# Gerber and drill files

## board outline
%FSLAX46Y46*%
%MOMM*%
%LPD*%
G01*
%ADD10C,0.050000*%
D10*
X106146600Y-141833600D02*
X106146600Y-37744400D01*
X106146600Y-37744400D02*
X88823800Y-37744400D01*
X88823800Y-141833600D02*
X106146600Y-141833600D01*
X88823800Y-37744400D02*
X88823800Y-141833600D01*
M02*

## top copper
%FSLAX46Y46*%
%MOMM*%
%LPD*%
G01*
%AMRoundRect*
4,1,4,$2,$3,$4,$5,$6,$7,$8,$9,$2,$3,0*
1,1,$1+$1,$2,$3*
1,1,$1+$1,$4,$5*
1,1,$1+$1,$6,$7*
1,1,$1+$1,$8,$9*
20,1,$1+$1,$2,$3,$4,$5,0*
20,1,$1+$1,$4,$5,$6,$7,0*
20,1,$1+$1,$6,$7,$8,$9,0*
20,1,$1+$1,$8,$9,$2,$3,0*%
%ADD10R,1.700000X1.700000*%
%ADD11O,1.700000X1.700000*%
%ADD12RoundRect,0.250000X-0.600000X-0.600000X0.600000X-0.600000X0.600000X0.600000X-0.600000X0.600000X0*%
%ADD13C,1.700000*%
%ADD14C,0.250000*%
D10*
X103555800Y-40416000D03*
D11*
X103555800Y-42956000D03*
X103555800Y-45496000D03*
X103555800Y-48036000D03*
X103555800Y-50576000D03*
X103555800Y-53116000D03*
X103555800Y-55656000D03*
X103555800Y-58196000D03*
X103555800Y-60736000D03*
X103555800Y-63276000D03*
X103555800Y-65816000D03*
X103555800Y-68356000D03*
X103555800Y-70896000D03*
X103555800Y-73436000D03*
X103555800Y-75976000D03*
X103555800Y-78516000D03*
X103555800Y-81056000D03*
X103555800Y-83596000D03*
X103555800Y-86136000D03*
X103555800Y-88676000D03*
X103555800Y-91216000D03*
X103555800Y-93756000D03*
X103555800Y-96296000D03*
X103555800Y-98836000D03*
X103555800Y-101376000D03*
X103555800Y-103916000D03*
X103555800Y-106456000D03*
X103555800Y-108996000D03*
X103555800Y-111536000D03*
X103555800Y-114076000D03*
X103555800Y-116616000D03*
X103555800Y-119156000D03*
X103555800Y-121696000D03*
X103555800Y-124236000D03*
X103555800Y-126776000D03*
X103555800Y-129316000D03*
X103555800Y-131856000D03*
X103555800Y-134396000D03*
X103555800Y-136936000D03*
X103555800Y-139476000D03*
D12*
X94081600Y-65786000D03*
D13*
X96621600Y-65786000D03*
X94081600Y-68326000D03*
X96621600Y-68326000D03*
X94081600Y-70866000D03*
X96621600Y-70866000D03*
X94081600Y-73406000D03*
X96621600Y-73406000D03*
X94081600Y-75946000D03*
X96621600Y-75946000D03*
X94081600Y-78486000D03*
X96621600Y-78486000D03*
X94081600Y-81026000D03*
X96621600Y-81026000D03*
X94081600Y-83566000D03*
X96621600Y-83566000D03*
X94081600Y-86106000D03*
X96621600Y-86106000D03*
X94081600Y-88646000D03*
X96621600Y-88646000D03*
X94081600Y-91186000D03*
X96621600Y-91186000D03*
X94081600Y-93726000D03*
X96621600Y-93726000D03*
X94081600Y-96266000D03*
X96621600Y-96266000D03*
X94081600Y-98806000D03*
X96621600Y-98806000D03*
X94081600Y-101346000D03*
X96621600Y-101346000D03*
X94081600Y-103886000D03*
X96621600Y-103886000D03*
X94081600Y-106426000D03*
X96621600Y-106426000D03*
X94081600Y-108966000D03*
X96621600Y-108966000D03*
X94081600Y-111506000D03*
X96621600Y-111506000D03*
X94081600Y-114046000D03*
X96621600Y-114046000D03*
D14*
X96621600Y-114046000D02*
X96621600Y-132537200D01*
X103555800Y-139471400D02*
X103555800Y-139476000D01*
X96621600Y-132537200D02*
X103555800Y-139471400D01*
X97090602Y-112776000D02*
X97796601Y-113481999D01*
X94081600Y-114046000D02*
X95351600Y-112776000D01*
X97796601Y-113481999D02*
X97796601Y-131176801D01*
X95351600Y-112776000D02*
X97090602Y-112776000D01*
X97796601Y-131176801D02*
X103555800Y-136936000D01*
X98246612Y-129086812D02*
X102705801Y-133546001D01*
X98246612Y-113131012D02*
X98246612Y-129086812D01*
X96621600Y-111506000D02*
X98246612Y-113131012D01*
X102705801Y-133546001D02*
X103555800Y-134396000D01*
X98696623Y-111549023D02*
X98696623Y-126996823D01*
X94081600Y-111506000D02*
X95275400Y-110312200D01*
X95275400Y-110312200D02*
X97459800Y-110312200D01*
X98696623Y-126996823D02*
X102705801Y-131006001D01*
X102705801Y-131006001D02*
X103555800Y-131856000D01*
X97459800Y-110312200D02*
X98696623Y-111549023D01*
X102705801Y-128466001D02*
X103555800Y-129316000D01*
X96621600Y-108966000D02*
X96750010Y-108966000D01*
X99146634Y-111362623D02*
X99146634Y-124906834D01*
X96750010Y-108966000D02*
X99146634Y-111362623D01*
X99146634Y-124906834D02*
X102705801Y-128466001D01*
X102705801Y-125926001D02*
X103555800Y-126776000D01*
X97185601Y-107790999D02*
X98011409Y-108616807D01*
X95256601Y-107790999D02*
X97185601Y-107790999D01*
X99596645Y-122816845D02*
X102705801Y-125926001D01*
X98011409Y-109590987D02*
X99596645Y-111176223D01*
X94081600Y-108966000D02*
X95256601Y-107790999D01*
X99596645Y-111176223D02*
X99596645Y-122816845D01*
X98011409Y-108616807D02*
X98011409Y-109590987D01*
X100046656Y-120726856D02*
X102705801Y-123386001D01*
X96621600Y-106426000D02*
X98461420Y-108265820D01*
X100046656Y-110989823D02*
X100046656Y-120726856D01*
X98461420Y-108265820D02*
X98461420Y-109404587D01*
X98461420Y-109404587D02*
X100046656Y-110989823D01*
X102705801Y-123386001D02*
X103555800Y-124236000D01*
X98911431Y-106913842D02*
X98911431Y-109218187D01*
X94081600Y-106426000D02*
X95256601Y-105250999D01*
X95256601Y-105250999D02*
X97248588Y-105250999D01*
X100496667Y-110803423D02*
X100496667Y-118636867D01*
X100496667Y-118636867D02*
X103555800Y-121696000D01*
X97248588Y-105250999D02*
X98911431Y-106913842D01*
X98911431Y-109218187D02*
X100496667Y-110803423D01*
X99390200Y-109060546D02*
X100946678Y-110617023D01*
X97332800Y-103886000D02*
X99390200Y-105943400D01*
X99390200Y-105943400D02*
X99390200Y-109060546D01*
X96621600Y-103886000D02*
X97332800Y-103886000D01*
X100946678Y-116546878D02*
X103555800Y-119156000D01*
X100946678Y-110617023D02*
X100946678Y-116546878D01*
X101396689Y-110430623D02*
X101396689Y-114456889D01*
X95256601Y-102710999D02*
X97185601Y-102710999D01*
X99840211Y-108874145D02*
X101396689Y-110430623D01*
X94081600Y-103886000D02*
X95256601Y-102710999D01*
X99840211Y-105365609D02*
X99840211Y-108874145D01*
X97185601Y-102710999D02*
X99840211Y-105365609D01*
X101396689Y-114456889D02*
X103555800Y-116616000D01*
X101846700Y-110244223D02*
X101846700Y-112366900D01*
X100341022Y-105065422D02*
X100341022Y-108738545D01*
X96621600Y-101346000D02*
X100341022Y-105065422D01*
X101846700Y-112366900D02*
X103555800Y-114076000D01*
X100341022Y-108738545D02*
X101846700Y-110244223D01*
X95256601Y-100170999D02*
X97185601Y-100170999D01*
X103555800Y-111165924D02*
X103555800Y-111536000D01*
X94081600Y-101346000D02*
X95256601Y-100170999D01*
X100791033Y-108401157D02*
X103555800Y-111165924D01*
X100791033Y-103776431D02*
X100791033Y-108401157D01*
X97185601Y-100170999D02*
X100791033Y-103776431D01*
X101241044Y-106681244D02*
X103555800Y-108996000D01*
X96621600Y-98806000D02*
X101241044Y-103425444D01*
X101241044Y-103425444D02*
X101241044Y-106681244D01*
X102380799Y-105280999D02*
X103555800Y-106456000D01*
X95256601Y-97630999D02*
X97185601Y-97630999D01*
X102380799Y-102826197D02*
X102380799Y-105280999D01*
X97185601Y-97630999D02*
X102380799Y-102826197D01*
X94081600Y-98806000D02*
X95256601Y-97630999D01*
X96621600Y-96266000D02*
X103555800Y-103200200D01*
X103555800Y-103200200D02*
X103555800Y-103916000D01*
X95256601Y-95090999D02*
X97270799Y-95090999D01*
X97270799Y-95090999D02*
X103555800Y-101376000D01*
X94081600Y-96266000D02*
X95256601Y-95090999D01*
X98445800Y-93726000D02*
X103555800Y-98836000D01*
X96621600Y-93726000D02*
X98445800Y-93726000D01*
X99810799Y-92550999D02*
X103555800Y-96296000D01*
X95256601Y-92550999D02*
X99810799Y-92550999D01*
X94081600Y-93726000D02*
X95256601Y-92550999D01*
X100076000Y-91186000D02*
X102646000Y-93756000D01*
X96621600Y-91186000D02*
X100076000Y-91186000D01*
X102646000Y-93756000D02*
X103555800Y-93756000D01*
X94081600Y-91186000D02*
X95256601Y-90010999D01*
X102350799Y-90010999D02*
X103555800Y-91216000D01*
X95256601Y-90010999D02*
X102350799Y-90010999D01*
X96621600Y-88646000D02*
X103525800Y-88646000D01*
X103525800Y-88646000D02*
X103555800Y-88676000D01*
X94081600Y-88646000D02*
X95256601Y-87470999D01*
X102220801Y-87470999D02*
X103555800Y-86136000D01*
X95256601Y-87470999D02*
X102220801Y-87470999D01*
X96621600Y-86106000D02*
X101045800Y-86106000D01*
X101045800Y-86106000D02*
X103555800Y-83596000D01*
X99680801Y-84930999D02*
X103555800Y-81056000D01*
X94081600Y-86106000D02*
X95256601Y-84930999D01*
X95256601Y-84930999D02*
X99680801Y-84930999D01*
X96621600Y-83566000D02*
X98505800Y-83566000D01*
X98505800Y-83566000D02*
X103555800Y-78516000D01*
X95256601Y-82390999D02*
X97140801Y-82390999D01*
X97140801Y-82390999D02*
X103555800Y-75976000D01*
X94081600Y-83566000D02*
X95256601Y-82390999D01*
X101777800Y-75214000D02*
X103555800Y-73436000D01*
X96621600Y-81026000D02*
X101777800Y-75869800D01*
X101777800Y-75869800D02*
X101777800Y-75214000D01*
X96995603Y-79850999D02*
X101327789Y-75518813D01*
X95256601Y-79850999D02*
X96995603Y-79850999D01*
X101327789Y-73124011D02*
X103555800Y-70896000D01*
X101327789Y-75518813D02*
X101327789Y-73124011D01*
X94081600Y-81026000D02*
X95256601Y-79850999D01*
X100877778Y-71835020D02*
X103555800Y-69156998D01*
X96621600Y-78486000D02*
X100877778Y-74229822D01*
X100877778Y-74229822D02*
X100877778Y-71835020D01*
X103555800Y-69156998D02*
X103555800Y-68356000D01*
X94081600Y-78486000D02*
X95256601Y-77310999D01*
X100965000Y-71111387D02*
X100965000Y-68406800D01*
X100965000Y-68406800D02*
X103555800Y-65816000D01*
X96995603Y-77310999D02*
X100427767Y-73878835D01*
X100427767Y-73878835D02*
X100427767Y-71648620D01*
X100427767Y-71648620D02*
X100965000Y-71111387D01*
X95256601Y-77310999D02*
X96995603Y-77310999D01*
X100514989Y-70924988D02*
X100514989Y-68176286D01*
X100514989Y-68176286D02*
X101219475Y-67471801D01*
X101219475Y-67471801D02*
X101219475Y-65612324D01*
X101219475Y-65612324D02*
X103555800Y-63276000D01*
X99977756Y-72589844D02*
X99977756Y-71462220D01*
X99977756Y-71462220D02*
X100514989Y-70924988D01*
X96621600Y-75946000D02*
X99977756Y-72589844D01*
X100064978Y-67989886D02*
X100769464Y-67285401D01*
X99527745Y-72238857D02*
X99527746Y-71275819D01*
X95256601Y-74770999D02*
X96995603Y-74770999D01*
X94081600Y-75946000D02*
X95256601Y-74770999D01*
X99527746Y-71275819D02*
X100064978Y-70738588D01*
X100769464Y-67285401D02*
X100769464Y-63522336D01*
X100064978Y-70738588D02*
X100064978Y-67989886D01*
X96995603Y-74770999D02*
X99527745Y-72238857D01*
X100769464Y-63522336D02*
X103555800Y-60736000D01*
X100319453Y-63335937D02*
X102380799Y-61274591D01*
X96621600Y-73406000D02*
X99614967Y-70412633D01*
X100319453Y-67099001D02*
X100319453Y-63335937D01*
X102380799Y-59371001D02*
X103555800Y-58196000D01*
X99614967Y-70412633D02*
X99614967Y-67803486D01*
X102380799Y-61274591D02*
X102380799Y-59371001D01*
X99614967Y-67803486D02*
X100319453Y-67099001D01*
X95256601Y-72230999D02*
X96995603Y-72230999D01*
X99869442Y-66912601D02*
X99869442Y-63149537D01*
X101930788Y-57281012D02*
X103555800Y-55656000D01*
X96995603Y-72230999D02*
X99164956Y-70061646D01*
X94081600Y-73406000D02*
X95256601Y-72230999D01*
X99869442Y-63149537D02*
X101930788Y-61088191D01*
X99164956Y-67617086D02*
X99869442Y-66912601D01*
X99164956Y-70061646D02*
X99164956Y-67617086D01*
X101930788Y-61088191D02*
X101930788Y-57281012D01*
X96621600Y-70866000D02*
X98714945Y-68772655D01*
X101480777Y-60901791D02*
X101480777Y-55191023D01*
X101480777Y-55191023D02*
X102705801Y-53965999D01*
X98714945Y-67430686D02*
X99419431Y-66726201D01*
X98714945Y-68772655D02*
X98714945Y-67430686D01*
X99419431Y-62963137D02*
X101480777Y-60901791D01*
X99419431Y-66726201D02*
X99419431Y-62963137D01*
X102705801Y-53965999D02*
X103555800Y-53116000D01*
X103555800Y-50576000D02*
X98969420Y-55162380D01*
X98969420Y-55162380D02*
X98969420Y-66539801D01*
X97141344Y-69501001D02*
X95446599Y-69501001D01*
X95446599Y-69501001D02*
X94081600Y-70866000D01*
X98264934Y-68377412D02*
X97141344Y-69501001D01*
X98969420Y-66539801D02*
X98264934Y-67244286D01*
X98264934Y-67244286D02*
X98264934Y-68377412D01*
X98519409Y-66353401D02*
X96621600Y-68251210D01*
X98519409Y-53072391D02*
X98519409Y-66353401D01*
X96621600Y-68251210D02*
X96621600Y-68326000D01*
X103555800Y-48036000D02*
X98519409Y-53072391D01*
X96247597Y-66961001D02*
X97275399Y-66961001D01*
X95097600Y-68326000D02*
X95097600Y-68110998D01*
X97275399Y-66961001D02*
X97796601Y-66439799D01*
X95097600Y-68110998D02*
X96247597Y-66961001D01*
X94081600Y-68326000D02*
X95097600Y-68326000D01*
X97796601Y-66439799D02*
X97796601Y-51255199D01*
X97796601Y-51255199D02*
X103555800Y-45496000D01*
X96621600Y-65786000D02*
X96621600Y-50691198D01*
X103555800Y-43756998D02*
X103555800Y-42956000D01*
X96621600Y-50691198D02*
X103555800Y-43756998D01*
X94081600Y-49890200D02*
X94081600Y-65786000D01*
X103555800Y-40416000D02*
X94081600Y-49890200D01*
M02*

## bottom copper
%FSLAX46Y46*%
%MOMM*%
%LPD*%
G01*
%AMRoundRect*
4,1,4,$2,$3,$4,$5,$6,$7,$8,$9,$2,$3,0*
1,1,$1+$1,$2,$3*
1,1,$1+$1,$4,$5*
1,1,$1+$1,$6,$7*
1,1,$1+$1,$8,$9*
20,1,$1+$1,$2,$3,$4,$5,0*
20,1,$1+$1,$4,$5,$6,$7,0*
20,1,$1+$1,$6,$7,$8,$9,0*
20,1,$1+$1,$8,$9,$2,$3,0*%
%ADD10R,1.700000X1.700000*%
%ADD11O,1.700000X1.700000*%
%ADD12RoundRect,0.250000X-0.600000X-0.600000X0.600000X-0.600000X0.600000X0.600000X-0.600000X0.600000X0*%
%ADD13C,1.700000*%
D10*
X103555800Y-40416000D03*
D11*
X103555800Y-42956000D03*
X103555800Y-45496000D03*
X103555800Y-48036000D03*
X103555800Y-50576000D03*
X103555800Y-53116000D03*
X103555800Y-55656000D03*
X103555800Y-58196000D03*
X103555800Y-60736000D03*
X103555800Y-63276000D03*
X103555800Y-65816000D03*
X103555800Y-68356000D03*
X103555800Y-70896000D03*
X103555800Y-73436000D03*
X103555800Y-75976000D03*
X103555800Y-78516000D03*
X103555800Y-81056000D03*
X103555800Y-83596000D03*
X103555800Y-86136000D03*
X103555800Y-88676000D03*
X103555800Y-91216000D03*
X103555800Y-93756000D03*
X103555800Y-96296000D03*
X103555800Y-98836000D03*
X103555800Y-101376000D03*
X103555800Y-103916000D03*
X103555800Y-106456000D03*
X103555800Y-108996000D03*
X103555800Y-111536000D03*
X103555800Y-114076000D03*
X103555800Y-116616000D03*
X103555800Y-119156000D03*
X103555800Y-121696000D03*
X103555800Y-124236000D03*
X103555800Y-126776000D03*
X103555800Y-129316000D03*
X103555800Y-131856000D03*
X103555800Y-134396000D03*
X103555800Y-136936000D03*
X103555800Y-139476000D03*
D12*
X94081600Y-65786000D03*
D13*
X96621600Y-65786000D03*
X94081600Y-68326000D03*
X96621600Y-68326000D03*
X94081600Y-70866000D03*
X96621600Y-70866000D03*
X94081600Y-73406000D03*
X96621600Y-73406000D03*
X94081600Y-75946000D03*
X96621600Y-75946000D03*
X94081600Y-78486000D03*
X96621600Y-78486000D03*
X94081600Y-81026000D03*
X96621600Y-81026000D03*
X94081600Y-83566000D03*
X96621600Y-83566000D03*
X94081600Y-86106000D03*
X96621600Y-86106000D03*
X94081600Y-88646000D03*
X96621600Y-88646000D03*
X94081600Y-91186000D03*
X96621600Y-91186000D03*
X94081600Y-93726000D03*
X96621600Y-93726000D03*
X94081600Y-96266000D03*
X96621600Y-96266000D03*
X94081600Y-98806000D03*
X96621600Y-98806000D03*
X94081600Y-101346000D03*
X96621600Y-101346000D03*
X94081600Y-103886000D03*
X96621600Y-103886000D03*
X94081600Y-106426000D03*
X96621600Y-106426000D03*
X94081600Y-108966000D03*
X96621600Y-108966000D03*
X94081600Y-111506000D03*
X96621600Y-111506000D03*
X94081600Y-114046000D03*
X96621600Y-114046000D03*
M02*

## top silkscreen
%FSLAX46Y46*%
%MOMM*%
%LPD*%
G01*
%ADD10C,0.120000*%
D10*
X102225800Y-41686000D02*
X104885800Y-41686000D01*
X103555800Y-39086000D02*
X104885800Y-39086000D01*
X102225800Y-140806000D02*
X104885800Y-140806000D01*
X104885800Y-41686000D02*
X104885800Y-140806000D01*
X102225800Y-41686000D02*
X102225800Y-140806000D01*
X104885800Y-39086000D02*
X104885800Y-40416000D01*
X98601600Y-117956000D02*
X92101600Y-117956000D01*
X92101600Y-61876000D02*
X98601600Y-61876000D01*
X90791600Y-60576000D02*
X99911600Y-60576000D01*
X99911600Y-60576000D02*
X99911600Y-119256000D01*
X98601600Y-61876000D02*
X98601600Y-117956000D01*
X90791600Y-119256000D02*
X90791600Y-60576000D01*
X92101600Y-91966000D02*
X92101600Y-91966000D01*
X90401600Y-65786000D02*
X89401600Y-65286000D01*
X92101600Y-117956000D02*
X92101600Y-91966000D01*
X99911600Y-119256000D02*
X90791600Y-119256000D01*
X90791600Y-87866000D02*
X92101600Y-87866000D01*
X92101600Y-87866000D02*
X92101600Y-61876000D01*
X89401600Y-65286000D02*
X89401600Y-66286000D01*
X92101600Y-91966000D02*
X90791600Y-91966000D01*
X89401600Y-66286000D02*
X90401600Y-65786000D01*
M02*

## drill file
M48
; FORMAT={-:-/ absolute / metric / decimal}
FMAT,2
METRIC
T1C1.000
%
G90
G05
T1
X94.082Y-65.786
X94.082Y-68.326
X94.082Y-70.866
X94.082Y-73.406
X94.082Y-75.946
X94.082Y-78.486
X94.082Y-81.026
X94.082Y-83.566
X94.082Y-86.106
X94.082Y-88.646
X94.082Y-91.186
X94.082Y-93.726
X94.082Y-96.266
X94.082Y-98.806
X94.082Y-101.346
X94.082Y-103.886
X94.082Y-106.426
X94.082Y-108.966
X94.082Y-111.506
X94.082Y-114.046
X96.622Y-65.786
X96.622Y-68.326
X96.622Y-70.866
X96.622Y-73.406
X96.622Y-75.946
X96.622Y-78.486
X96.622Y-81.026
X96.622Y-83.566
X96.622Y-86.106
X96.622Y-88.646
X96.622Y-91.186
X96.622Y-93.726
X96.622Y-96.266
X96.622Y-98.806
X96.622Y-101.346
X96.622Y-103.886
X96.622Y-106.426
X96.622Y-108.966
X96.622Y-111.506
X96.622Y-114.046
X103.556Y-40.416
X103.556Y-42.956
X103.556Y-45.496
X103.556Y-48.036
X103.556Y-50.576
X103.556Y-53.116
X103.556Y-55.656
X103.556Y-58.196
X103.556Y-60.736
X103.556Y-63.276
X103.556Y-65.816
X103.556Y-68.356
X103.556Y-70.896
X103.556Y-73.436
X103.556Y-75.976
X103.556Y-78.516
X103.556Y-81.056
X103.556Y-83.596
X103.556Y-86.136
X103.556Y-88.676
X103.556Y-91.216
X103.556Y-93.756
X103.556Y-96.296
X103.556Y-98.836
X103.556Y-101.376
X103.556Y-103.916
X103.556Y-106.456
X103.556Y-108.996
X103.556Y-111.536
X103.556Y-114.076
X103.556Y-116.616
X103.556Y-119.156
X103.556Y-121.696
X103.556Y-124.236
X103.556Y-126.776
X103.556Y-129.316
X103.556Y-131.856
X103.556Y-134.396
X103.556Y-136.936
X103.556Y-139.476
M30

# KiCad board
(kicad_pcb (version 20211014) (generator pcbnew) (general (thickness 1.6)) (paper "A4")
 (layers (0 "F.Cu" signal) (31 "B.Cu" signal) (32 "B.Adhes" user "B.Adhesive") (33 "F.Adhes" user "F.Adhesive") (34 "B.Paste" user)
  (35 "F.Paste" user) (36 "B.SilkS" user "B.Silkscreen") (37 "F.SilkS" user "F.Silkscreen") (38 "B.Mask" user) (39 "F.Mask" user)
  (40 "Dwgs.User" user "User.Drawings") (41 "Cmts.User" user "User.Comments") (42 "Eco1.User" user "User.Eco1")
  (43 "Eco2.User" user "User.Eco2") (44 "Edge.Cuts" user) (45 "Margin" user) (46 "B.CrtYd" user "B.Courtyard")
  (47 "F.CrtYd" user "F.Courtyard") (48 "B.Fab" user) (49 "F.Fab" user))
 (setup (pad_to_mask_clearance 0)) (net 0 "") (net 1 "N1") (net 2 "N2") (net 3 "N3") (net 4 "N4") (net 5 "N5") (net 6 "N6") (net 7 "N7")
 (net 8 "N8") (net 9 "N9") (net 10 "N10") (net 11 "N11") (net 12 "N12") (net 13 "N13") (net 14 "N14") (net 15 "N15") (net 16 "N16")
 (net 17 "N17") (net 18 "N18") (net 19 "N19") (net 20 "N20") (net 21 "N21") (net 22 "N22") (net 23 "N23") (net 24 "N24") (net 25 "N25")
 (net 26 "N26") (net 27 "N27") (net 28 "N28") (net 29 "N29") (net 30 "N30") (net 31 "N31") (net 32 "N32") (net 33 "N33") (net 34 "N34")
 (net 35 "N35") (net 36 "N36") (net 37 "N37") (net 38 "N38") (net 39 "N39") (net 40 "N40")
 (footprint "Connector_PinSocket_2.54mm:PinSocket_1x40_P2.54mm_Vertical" (layer "F.Cu") (at 103.5558 40.416)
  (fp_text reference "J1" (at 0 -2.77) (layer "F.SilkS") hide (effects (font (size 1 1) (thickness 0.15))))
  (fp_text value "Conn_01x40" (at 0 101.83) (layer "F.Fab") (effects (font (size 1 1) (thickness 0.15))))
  (fp_line (start -1.33 1.27) (end 1.33 1.27) (layer "F.SilkS") (width 0.12))
  (fp_line (start 0 -1.33) (end 1.33 -1.33) (layer "F.SilkS") (width 0.12))
  (fp_line (start -1.33 100.39) (end 1.33 100.39) (layer "F.SilkS") (width 0.12))
  (fp_line (start 1.33 1.27) (end 1.33 100.39) (layer "F.SilkS") (width 0.12))
  (fp_line (start -1.33 1.27) (end -1.33 100.39) (layer "F.SilkS") (width 0.12))
  (fp_line (start 1.33 -1.33) (end 1.33 0) (layer "F.SilkS") (width 0.12))
  (pad "1" thru_hole rect locked (at 0 0) (size 1.7 1.7) (drill 1) (layers *.Cu *.Mask) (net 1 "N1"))
  (pad "2" thru_hole oval locked (at 0 2.54) (size 1.7 1.7) (drill 1) (layers *.Cu *.Mask) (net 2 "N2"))
  (pad "3" thru_hole oval locked (at 0 5.08) (size 1.7 1.7) (drill 1) (layers *.Cu *.Mask) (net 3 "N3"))
  (pad "4" thru_hole oval locked (at 0 7.62) (size 1.7 1.7) (drill 1) (layers *.Cu *.Mask) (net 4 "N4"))
  (pad "5" thru_hole oval locked (at 0 10.16) (size 1.7 1.7) (drill 1) (layers *.Cu *.Mask) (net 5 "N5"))
  (pad "6" thru_hole oval locked (at 0 12.7) (size 1.7 1.7) (drill 1) (layers *.Cu *.Mask) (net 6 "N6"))
  (pad "7" thru_hole oval locked (at 0 15.24) (size 1.7 1.7) (drill 1) (layers *.Cu *.Mask) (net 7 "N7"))
  (pad "8" thru_hole oval locked (at 0 17.78) (size 1.7 1.7) (drill 1) (layers *.Cu *.Mask) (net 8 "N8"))
  (pad "9" thru_hole oval locked (at 0 20.32) (size 1.7 1.7) (drill 1) (layers *.Cu *.Mask) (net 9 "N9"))
  (pad "10" thru_hole oval locked (at 0 22.86) (size 1.7 1.7) (drill 1) (layers *.Cu *.Mask) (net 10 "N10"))
  (pad "11" thru_hole oval locked (at 0 25.4) (size 1.7 1.7) (drill 1) (layers *.Cu *.Mask) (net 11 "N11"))
  (pad "12" thru_hole oval locked (at 0 27.94) (size 1.7 1.7) (drill 1) (layers *.Cu *.Mask) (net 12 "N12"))
  (pad "13" thru_hole oval locked (at 0 30.48) (size 1.7 1.7) (drill 1) (layers *.Cu *.Mask) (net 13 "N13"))
  (pad "14" thru_hole oval locked (at 0 33.02) (size 1.7 1.7) (drill 1) (layers *.Cu *.Mask) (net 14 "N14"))
  (pad "15" thru_hole oval locked (at 0 35.56) (size 1.7 1.7) (drill 1) (layers *.Cu *.Mask) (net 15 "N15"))
  (pad "16" thru_hole oval locked (at 0 38.1) (size 1.7 1.7) (drill 1) (layers *.Cu *.Mask) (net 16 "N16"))
  (pad "17" thru_hole oval locked (at 0 40.64) (size 1.7 1.7) (drill 1) (layers *.Cu *.Mask) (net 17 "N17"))
  (pad "18" thru_hole oval locked (at 0 43.18) (size 1.7 1.7) (drill 1) (layers *.Cu *.Mask) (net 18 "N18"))
  (pad "19" thru_hole oval locked (at 0 45.72) (size 1.7 1.7) (drill 1) (layers *.Cu *.Mask) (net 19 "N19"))
  (pad "20" thru_hole oval locked (at 0 48.26) (size 1.7 1.7) (drill 1) (layers *.Cu *.Mask) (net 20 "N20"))
  (pad "21" thru_hole oval locked (at 0 50.8) (size 1.7 1.7) (drill 1) (layers *.Cu *.Mask) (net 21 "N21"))
  (pad "22" thru_hole oval locked (at 0 53.34) (size 1.7 1.7) (drill 1) (layers *.Cu *.Mask) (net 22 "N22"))
  (pad "23" thru_hole oval locked (at 0 55.88) (size 1.7 1.7) (drill 1) (layers *.Cu *.Mask) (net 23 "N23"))
  (pad "24" thru_hole oval locked (at 0 58.42) (size 1.7 1.7) (drill 1) (layers *.Cu *.Mask) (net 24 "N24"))
  (pad "25" thru_hole oval locked (at 0 60.96) (size 1.7 1.7) (drill 1) (layers *.Cu *.Mask) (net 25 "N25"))
  (pad "26" thru_hole oval locked (at 0 63.5) (size 1.7 1.7) (drill 1) (layers *.Cu *.Mask) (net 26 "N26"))
  (pad "27" thru_hole oval locked (at 0 66.04) (size 1.7 1.7) (drill 1) (layers *.Cu *.Mask) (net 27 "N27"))
  (pad "28" thru_hole oval locked (at 0 68.58) (size 1.7 1.7) (drill 1) (layers *.Cu *.Mask) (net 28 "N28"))
  (pad "29" thru_hole oval locked (at 0 71.12) (size 1.7 1.7) (drill 1) (layers *.Cu *.Mask) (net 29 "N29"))
  (pad "30" thru_hole oval locked (at 0 73.66) (size 1.7 1.7) (drill 1) (layers *.Cu *.Mask) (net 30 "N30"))
  (pad "31" thru_hole oval locked (at 0 76.2) (size 1.7 1.7) (drill 1) (layers *.Cu *.Mask) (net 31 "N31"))
  (pad "32" thru_hole oval locked (at 0 78.74) (size 1.7 1.7) (drill 1) (layers *.Cu *.Mask) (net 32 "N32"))
  (pad "33" thru_hole oval locked (at 0 81.28) (size 1.7 1.7) (drill 1) (layers *.Cu *.Mask) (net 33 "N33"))
  (pad "34" thru_hole oval locked (at 0 83.82) (size 1.7 1.7) (drill 1) (layers *.Cu *.Mask) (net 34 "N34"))
  (pad "35" thru_hole oval locked (at 0 86.36) (size 1.7 1.7) (drill 1) (layers *.Cu *.Mask) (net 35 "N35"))
  (pad "36" thru_hole oval locked (at 0 88.9) (size 1.7 1.7) (drill 1) (layers *.Cu *.Mask) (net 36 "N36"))
  (pad "37" thru_hole oval locked (at 0 91.44) (size 1.7 1.7) (drill 1) (layers *.Cu *.Mask) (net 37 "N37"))
  (pad "38" thru_hole oval locked (at 0 93.98) (size 1.7 1.7) (drill 1) (layers *.Cu *.Mask) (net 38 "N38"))
  (pad "39" thru_hole oval locked (at 0 96.52) (size 1.7 1.7) (drill 1) (layers *.Cu *.Mask) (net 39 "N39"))
  (pad "40" thru_hole oval locked (at 0 99.06) (size 1.7 1.7) (drill 1) (layers *.Cu *.Mask) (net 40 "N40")))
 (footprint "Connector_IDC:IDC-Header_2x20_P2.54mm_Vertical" (layer "F.Cu") (at 94.0816 65.786)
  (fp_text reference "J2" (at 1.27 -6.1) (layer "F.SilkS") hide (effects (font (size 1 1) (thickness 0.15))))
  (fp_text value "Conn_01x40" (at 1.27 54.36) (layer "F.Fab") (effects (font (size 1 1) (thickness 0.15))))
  (fp_line (start 4.52 52.17) (end -1.98 52.17) (layer "F.SilkS") (width 0.12))
  (fp_line (start -1.98 -3.91) (end 4.52 -3.91) (layer "F.SilkS") (width 0.12))
  (fp_line (start -3.29 -5.21) (end 5.83 -5.21) (layer "F.SilkS") (width 0.12))
  (fp_line (start 5.83 -5.21) (end 5.83 53.47) (layer "F.SilkS") (width 0.12))
  (fp_line (start 4.52 -3.91) (end 4.52 52.17) (layer "F.SilkS") (width 0.12))
  (fp_line (start -3.29 53.47) (end -3.29 -5.21) (layer "F.SilkS") (width 0.12))
  (fp_line (start -1.98 26.18) (end -1.98 26.18) (layer "F.SilkS") (width 0.12))
  (fp_line (start -3.68 0) (end -4.68 -0.5) (layer "F.SilkS") (width 0.12))
  (fp_line (start -1.98 52.17) (end -1.98 26.18) (layer "F.SilkS") (width 0.12))
  (fp_line (start 5.83 53.47) (end -3.29 53.47) (layer "F.SilkS") (width 0.12))
  (fp_line (start -3.29 22.08) (end -1.98 22.08) (layer "F.SilkS") (width 0.12))
  (fp_line (start -1.98 22.08) (end -1.98 -3.91) (layer "F.SilkS") (width 0.12))
  (fp_line (start -4.68 -0.5) (end -4.68 0.5) (layer "F.SilkS") (width 0.12))
  (fp_line (start -1.98 26.18) (end -3.29 26.18) (layer "F.SilkS") (width 0.12))
  (fp_line (start -4.68 0.5) (end -3.68 0) (layer "F.SilkS") (width 0.12))
  (pad "1" thru_hole roundrect locked (at 0 0) (size 1.7 1.7) (drill 1) (layers *.Cu *.Mask) (roundrect_rratio 0.1470588235) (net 1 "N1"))
  (pad "2" thru_hole circle locked (at 2.54 0) (size 1.7 1.7) (drill 1) (layers *.Cu *.Mask) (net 2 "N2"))
  (pad "3" thru_hole circle locked (at 0 2.54) (size 1.7 1.7) (drill 1) (layers *.Cu *.Mask) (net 3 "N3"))
  (pad "4" thru_hole circle locked (at 2.54 2.54) (size 1.7 1.7) (drill 1) (layers *.Cu *.Mask) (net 4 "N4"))
  (pad "5" thru_hole circle locked (at 0 5.08) (size 1.7 1.7) (drill 1) (layers *.Cu *.Mask) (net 5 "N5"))
  (pad "6" thru_hole circle locked (at 2.54 5.08) (size 1.7 1.7) (drill 1) (layers *.Cu *.Mask) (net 6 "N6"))
  (pad "7" thru_hole circle locked (at 0 7.62) (size 1.7 1.7) (drill 1) (layers *.Cu *.Mask) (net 7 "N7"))
  (pad "8" thru_hole circle locked (at 2.54 7.62) (size 1.7 1.7) (drill 1) (layers *.Cu *.Mask) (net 8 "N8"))
  (pad "9" thru_hole circle locked (at 0 10.16) (size 1.7 1.7) (drill 1) (layers *.Cu *.Mask) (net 9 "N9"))
  (pad "10" thru_hole circle locked (at 2.54 10.16) (size 1.7 1.7) (drill 1) (layers *.Cu *.Mask) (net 10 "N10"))
  (pad "11" thru_hole circle locked (at 0 12.7) (size 1.7 1.7) (drill 1) (layers *.Cu *.Mask) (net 11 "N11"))
  (pad "12" thru_hole circle locked (at 2.54 12.7) (size 1.7 1.7) (drill 1) (layers *.Cu *.Mask) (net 12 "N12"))
  (pad "13" thru_hole circle locked (at 0 15.24) (size 1.7 1.7) (drill 1) (layers *.Cu *.Mask) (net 13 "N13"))
  (pad "14" thru_hole circle locked (at 2.54 15.24) (size 1.7 1.7) (drill 1) (layers *.Cu *.Mask) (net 14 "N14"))
  (pad "15" thru_hole circle locked (at 0 17.78) (size 1.7 1.7) (drill 1) (layers *.Cu *.Mask) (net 15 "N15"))
  (pad "16" thru_hole circle locked (at 2.54 17.78) (size 1.7 1.7) (drill 1) (layers *.Cu *.Mask) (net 16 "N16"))
  (pad "17" thru_hole circle locked (at 0 20.32) (size 1.7 1.7) (drill 1) (layers *.Cu *.Mask) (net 17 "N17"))
  (pad "18" thru_hole circle locked (at 2.54 20.32) (size 1.7 1.7) (drill 1) (layers *.Cu *.Mask) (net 18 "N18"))
  (pad "19" thru_hole circle locked (at 0 22.86) (size 1.7 1.7) (drill 1) (layers *.Cu *.Mask) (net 19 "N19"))
  (pad "20" thru_hole circle locked (at 2.54 22.86) (size 1.7 1.7) (drill 1) (layers *.Cu *.Mask) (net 20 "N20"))
  (pad "21" thru_hole circle locked (at 0 25.4) (size 1.7 1.7) (drill 1) (layers *.Cu *.Mask) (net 21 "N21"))
  (pad "22" thru_hole circle locked (at 2.54 25.4) (size 1.7 1.7) (drill 1) (layers *.Cu *.Mask) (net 22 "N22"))
  (pad "23" thru_hole circle locked (at 0 27.94) (size 1.7 1.7) (drill 1) (layers *.Cu *.Mask) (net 23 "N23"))
  (pad "24" thru_hole circle locked (at 2.54 27.94) (size 1.7 1.7) (drill 1) (layers *.Cu *.Mask) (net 24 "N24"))
  (pad "25" thru_hole circle locked (at 0 30.48) (size 1.7 1.7) (drill 1) (layers *.Cu *.Mask) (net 25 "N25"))
  (pad "26" thru_hole circle locked (at 2.54 30.48) (size 1.7 1.7) (drill 1) (layers *.Cu *.Mask) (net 26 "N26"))
  (pad "27" thru_hole circle locked (at 0 33.02) (size 1.7 1.7) (drill 1) (layers *.Cu *.Mask) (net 27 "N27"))
  (pad "28" thru_hole circle locked (at 2.54 33.02) (size 1.7 1.7) (drill 1) (layers *.Cu *.Mask) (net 28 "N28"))
  (pad "29" thru_hole circle locked (at 0 35.56) (size 1.7 1.7) (drill 1) (layers *.Cu *.Mask) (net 29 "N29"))
  (pad "30" thru_hole circle locked (at 2.54 35.56) (size 1.7 1.7) (drill 1) (layers *.Cu *.Mask) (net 30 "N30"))
  (pad "31" thru_hole circle locked (at 0 38.1) (size 1.7 1.7) (drill 1) (layers *.Cu *.Mask) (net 31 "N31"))
  (pad "32" thru_hole circle locked (at 2.54 38.1) (size 1.7 1.7) (drill 1) (layers *.Cu *.Mask) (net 32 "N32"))
  (pad "33" thru_hole circle locked (at 0 40.64) (size 1.7 1.7) (drill 1) (layers *.Cu *.Mask) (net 33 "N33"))
  (pad "34" thru_hole circle locked (at 2.54 40.64) (size 1.7 1.7) (drill 1) (layers *.Cu *.Mask) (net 34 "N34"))
  (pad "35" thru_hole circle locked (at 0 43.18) (size 1.7 1.7) (drill 1) (layers *.Cu *.Mask) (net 35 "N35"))
  (pad "36" thru_hole circle locked (at 2.54 43.18) (size 1.7 1.7) (drill 1) (layers *.Cu *.Mask) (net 36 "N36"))
  (pad "37" thru_hole circle locked (at 0 45.72) (size 1.7 1.7) (drill 1) (layers *.Cu *.Mask) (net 37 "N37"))
  (pad "38" thru_hole circle locked (at 2.54 45.72) (size 1.7 1.7) (drill 1) (layers *.Cu *.Mask) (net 38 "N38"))
  (pad "39" thru_hole circle locked (at 0 48.26) (size 1.7 1.7) (drill 1) (layers *.Cu *.Mask) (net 39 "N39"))
  (pad "40" thru_hole circle locked (at 2.54 48.26) (size 1.7 1.7) (drill 1) (layers *.Cu *.Mask) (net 40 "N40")))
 (gr_line (start 106.1466 141.8336) (end 106.1466 37.7444) (layer "Edge.Cuts") (width 0.05))
 (gr_line (start 106.1466 37.7444) (end 88.8238 37.7444) (layer "Edge.Cuts") (width 0.05))
 (gr_line (start 88.8238 141.8336) (end 106.1466 141.8336) (layer "Edge.Cuts") (width 0.05))
 (gr_line (start 88.8238 37.7444) (end 88.8238 141.8336) (layer "Edge.Cuts") (width 0.05))
 (segment (start 96.6216 114.046) (end 96.6216 132.5372) (width 0.25) (layer "F.Cu") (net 40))
 (segment (start 103.5558 139.4714) (end 103.5558 139.476) (width 0.25) (layer "F.Cu") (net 40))
 (segment (start 96.6216 132.5372) (end 103.5558 139.4714) (width 0.25) (layer "F.Cu") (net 40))
 (segment (start 97.090602 112.776) (end 97.796601 113.481999) (width 0.25) (layer "F.Cu") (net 39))
 (segment (start 94.0816 114.046) (end 95.3516 112.776) (width 0.25) (layer "F.Cu") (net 39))
 (segment (start 97.796601 113.481999) (end 97.796601 131.176801) (width 0.25) (layer "F.Cu") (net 39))
 (segment (start 95.3516 112.776) (end 97.090602 112.776) (width 0.25) (layer "F.Cu") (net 39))
 (segment (start 97.796601 131.176801) (end 103.5558 136.936) (width 0.25) (layer "F.Cu") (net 39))
 (segment (start 98.246612 129.086812) (end 102.705801 133.546001) (width 0.25) (layer "F.Cu") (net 38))
 (segment (start 98.246612 113.131012) (end 98.246612 129.086812) (width 0.25) (layer "F.Cu") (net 38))
 (segment (start 96.6216 111.506) (end 98.246612 113.131012) (width 0.25) (layer "F.Cu") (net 38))
 (segment (start 102.705801 133.546001) (end 103.5558 134.396) (width 0.25) (layer "F.Cu") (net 38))
 (segment (start 98.696623 111.549023) (end 98.696623 126.996823) (width 0.25) (layer "F.Cu") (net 37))
 (segment (start 94.0816 111.506) (end 95.2754 110.3122) (width 0.25) (layer "F.Cu") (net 37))
 (segment (start 95.2754 110.3122) (end 97.4598 110.3122) (width 0.25) (layer "F.Cu") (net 37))
 (segment (start 98.696623 126.996823) (end 102.705801 131.006001) (width 0.25) (layer "F.Cu") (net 37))
 (segment (start 102.705801 131.006001) (end 103.5558 131.856) (width 0.25) (layer "F.Cu") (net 37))
 (segment (start 97.4598 110.3122) (end 98.696623 111.549023) (width 0.25) (layer "F.Cu") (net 37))
 (segment (start 102.705801 128.466001) (end 103.5558 129.316) (width 0.25) (layer "F.Cu") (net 36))
 (segment (start 96.6216 108.966) (end 96.75001 108.966) (width 0.25) (layer "F.Cu") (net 36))
 (segment (start 99.146634 111.362623) (end 99.146634 124.906834) (width 0.25) (layer "F.Cu") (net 36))
 (segment (start 96.75001 108.966) (end 99.146634 111.362623) (width 0.25) (layer "F.Cu") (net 36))
 (segment (start 99.146634 124.906834) (end 102.705801 128.466001) (width 0.25) (layer "F.Cu") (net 36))
 (segment (start 102.705801 125.926001) (end 103.5558 126.776) (width 0.25) (layer "F.Cu") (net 35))
 (segment (start 97.185601 107.790999) (end 98.011409 108.616807) (width 0.25) (layer "F.Cu") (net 35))
 (segment (start 95.256601 107.790999) (end 97.185601 107.790999) (width 0.25) (layer "F.Cu") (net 35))
 (segment (start 99.596645 122.816845) (end 102.705801 125.926001) (width 0.25) (layer "F.Cu") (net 35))
 (segment (start 98.011409 109.590987) (end 99.596645 111.176223) (width 0.25) (layer "F.Cu") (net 35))
 (segment (start 94.0816 108.966) (end 95.256601 107.790999) (width 0.25) (layer "F.Cu") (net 35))
 (segment (start 99.596645 111.176223) (end 99.596645 122.816845) (width 0.25) (layer "F.Cu") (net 35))
 (segment (start 98.011409 108.616807) (end 98.011409 109.590987) (width 0.25) (layer "F.Cu") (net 35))
 (segment (start 100.046656 120.726856) (end 102.705801 123.386001) (width 0.25) (layer "F.Cu") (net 34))
 (segment (start 96.6216 106.426) (end 98.46142 108.26582) (width 0.25) (layer "F.Cu") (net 34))
 (segment (start 100.046656 110.989823) (end 100.046656 120.726856) (width 0.25) (layer "F.Cu") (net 34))
 (segment (start 98.46142 108.26582) (end 98.46142 109.404587) (width 0.25) (layer "F.Cu") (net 34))
 (segment (start 98.46142 109.404587) (end 100.046656 110.989823) (width 0.25) (layer "F.Cu") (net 34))
 (segment (start 102.705801 123.386001) (end 103.5558 124.236) (width 0.25) (layer "F.Cu") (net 34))
 (segment (start 98.911431 106.913842) (end 98.911431 109.218187) (width 0.25) (layer "F.Cu") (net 33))
 (segment (start 94.0816 106.426) (end 95.256601 105.250999) (width 0.25) (layer "F.Cu") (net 33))
 (segment (start 95.256601 105.250999) (end 97.248588 105.250999) (width 0.25) (layer "F.Cu") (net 33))
 (segment (start 100.496667 110.803423) (end 100.496667 118.636867) (width 0.25) (layer "F.Cu") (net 33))
 (segment (start 100.496667 118.636867) (end 103.5558 121.696) (width 0.25) (layer "F.Cu") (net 33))
 (segment (start 97.248588 105.250999) (end 98.911431 106.913842) (width 0.25) (layer "F.Cu") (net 33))
 (segment (start 98.911431 109.218187) (end 100.496667 110.803423) (width 0.25) (layer "F.Cu") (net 33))
 (segment (start 99.3902 109.060546) (end 100.946678 110.617023) (width 0.25) (layer "F.Cu") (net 32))
 (segment (start 97.3328 103.886) (end 99.3902 105.9434) (width 0.25) (layer "F.Cu") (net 32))
 (segment (start 99.3902 105.9434) (end 99.3902 109.060546) (width 0.25) (layer "F.Cu") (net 32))
 (segment (start 96.6216 103.886) (end 97.3328 103.886) (width 0.25) (layer "F.Cu") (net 32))
 (segment (start 100.946678 116.546878) (end 103.5558 119.156) (width 0.25) (layer "F.Cu") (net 32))
 (segment (start 100.946678 110.617023) (end 100.946678 116.546878) (width 0.25) (layer "F.Cu") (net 32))
 (segment (start 101.396689 110.430623) (end 101.396689 114.456889) (width 0.25) (layer "F.Cu") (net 31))
 (segment (start 95.256601 102.710999) (end 97.185601 102.710999) (width 0.25) (layer "F.Cu") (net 31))
 (segment (start 99.840211 108.874145) (end 101.396689 110.430623) (width 0.25) (layer "F.Cu") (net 31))
 (segment (start 94.0816 103.886) (end 95.256601 102.710999) (width 0.25) (layer "F.Cu") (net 31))
 (segment (start 99.840211 105.365609) (end 99.840211 108.874145) (width 0.25) (layer "F.Cu") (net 31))
 (segment (start 97.185601 102.710999) (end 99.840211 105.365609) (width 0.25) (layer "F.Cu") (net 31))
 (segment (start 101.396689 114.456889) (end 103.5558 116.616) (width 0.25) (layer "F.Cu") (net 31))
 (segment (start 101.8467 110.244223) (end 101.8467 112.3669) (width 0.25) (layer "F.Cu") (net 30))
 (segment (start 100.341022 105.065422) (end 100.341022 108.738545) (width 0.25) (layer "F.Cu") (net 30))
 (segment (start 96.6216 101.346) (end 100.341022 105.065422) (width 0.25) (layer "F.Cu") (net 30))
 (segment (start 101.8467 112.3669) (end 103.5558 114.076) (width 0.25) (layer "F.Cu") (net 30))
 (segment (start 100.341022 108.738545) (end 101.8467 110.244223) (width 0.25) (layer "F.Cu") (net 30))
 (segment (start 95.256601 100.170999) (end 97.185601 100.170999) (width 0.25) (layer "F.Cu") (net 29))
 (segment (start 103.5558 111.165924) (end 103.5558 111.536) (width 0.25) (layer "F.Cu") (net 29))
 (segment (start 94.0816 101.346) (end 95.256601 100.170999) (width 0.25) (layer "F.Cu") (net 29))
 (segment (start 100.791033 108.401157) (end 103.5558 111.165924) (width 0.25) (layer "F.Cu") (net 29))
 (segment (start 100.791033 103.776431) (end 100.791033 108.401157) (width 0.25) (layer "F.Cu") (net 29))
 (segment (start 97.185601 100.170999) (end 100.791033 103.776431) (width 0.25) (layer "F.Cu") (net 29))
 (segment (start 101.241044 106.681244) (end 103.5558 108.996) (width 0.25) (layer "F.Cu") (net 28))
 (segment (start 96.6216 98.806) (end 101.241044 103.425444) (width 0.25) (layer "F.Cu") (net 28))
 (segment (start 101.241044 103.425444) (end 101.241044 106.681244) (width 0.25) (layer "F.Cu") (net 28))
 (segment (start 102.380799 105.280999) (end 103.5558 106.456) (width 0.25) (layer "F.Cu") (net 27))
 (segment (start 95.256601 97.630999) (end 97.185601 97.630999) (width 0.25) (layer "F.Cu") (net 27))
 (segment (start 102.380799 102.826197) (end 102.380799 105.280999) (width 0.25) (layer "F.Cu") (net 27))
 (segment (start 97.185601 97.630999) (end 102.380799 102.826197) (width 0.25) (layer "F.Cu") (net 27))
 (segment (start 94.0816 98.806) (end 95.256601 97.630999) (width 0.25) (layer "F.Cu") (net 27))
 (segment (start 96.6216 96.266) (end 103.5558 103.2002) (width 0.25) (layer "F.Cu") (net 26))
 (segment (start 103.5558 103.2002) (end 103.5558 103.916) (width 0.25) (layer "F.Cu") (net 26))
 (segment (start 95.256601 95.090999) (end 97.270799 95.090999) (width 0.25) (layer "F.Cu") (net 25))
 (segment (start 97.270799 95.090999) (end 103.5558 101.376) (width 0.25) (layer "F.Cu") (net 25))
 (segment (start 94.0816 96.266) (end 95.256601 95.090999) (width 0.25) (layer "F.Cu") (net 25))
 (segment (start 98.4458 93.726) (end 103.5558 98.836) (width 0.25) (layer "F.Cu") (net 24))
 (segment (start 96.6216 93.726) (end 98.4458 93.726) (width 0.25) (layer "F.Cu") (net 24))
 (segment (start 99.810799 92.550999) (end 103.5558 96.296) (width 0.25) (layer "F.Cu") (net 23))
 (segment (start 95.256601 92.550999) (end 99.810799 92.550999) (width 0.25) (layer "F.Cu") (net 23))
 (segment (start 94.0816 93.726) (end 95.256601 92.550999) (width 0.25) (layer "F.Cu") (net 23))
 (segment (start 100.076 91.186) (end 102.646 93.756) (width 0.25) (layer "F.Cu") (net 22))
 (segment (start 96.6216 91.186) (end 100.076 91.186) (width 0.25) (layer "F.Cu") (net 22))
 (segment (start 102.646 93.756) (end 103.5558 93.756) (width 0.25) (layer "F.Cu") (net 22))
 (segment (start 94.0816 91.186) (end 95.256601 90.010999) (width 0.25) (layer "F.Cu") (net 21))
 (segment (start 102.350799 90.010999) (end 103.5558 91.216) (width 0.25) (layer "F.Cu") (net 21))
 (segment (start 95.256601 90.010999) (end 102.350799 90.010999) (width 0.25) (layer "F.Cu") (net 21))
 (segment (start 96.6216 88.646) (end 103.5258 88.646) (width 0.25) (layer "F.Cu") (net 20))
 (segment (start 103.5258 88.646) (end 103.5558 88.676) (width 0.25) (layer "F.Cu") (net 20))
 (segment (start 94.0816 88.646) (end 95.256601 87.470999) (width 0.25) (layer "F.Cu") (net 19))
 (segment (start 102.220801 87.470999) (end 103.5558 86.136) (width 0.25) (layer "F.Cu") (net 19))
 (segment (start 95.256601 87.470999) (end 102.220801 87.470999) (width 0.25) (layer "F.Cu") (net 19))
 (segment (start 96.6216 86.106) (end 101.0458 86.106) (width 0.25) (layer "F.Cu") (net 18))
 (segment (start 101.0458 86.106) (end 103.5558 83.596) (width 0.25) (layer "F.Cu") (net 18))
 (segment (start 99.680801 84.930999) (end 103.5558 81.056) (width 0.25) (layer "F.Cu") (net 17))
 (segment (start 94.0816 86.106) (end 95.256601 84.930999) (width 0.25) (layer "F.Cu") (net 17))
 (segment (start 95.256601 84.930999) (end 99.680801 84.930999) (width 0.25) (layer "F.Cu") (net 17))
 (segment (start 96.6216 83.566) (end 98.5058 83.566) (width 0.25) (layer "F.Cu") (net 16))
 (segment (start 98.5058 83.566) (end 103.5558 78.516) (width 0.25) (layer "F.Cu") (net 16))
 (segment (start 95.256601 82.390999) (end 97.140801 82.390999) (width 0.25) (layer "F.Cu") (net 15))
 (segment (start 97.140801 82.390999) (end 103.5558 75.976) (width 0.25) (layer "F.Cu") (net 15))
 (segment (start 94.0816 83.566) (end 95.256601 82.390999) (width 0.25) (layer "F.Cu") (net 15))
 (segment (start 101.7778 75.214) (end 103.5558 73.436) (width 0.25) (layer "F.Cu") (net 14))
 (segment (start 96.6216 81.026) (end 101.7778 75.8698) (width 0.25) (layer "F.Cu") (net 14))
 (segment (start 101.7778 75.8698) (end 101.7778 75.214) (width 0.25) (layer "F.Cu") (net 14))
 (segment (start 96.995603 79.850999) (end 101.327789 75.518813) (width 0.25) (layer "F.Cu") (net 13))
 (segment (start 95.256601 79.850999) (end 96.995603 79.850999) (width 0.25) (layer "F.Cu") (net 13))
 (segment (start 101.327789 73.124011) (end 103.5558 70.896) (width 0.25) (layer "F.Cu") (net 13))
 (segment (start 101.327789 75.518813) (end 101.327789 73.124011) (width 0.25) (layer "F.Cu") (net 13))
 (segment (start 94.0816 81.026) (end 95.256601 79.850999) (width 0.25) (layer "F.Cu") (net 13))
 (segment (start 100.877778 71.83502) (end 103.5558 69.156998) (width 0.25) (layer "F.Cu") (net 12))
 (segment (start 96.6216 78.486) (end 100.877778 74.229822) (width 0.25) (layer "F.Cu") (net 12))
 (segment (start 100.877778 74.229822) (end 100.877778 71.83502) (width 0.25) (layer "F.Cu") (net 12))
 (segment (start 103.5558 69.156998) (end 103.5558 68.356) (width 0.25) (layer "F.Cu") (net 12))
 (segment (start 94.0816 78.486) (end 95.256601 77.310999) (width 0.25) (layer "F.Cu") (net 11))
 (segment (start 100.965 71.111387) (end 100.965 68.4068) (width 0.25) (layer "F.Cu") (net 11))
 (segment (start 100.965 68.4068) (end 103.5558 65.816) (width 0.25) (layer "F.Cu") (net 11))
 (segment (start 96.995603 77.310999) (end 100.427767 73.878835) (width 0.25) (layer "F.Cu") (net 11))
 (segment (start 100.427767 73.878835) (end 100.427767 71.64862) (width 0.25) (layer "F.Cu") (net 11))
 (segment (start 100.427767 71.64862) (end 100.965 71.111387) (width 0.25) (layer "F.Cu") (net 11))
 (segment (start 95.256601 77.310999) (end 96.995603 77.310999) (width 0.25) (layer "F.Cu") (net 11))
 (segment (start 100.514989 70.924988) (end 100.514989 68.176286) (width 0.25) (layer "F.Cu") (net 10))
 (segment (start 100.514989 68.176286) (end 101.219475 67.471801) (width 0.25) (layer "F.Cu") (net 10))
 (segment (start 101.219475 67.471801) (end 101.219475 65.612324) (width 0.25) (layer "F.Cu") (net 10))
 (segment (start 101.219475 65.612324) (end 103.5558 63.276) (width 0.25) (layer "F.Cu") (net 10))
 (segment (start 99.977756 72.589844) (end 99.977756 71.46222) (width 0.25) (layer "F.Cu") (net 10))
 (segment (start 99.977756 71.46222) (end 100.514989 70.924988) (width 0.25) (layer "F.Cu") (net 10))
 (segment (start 96.6216 75.946) (end 99.977756 72.589844) (width 0.25) (layer "F.Cu") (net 10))
 (segment (start 100.064978 67.989886) (end 100.769464 67.285401) (width 0.25) (layer "F.Cu") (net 9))
 (segment (start 99.527745 72.238857) (end 99.527746 71.275819) (width 0.25) (layer "F.Cu") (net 9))
 (segment (start 95.256601 74.770999) (end 96.995603 74.770999) (width 0.25) (layer "F.Cu") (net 9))
 (segment (start 94.0816 75.946) (end 95.256601 74.770999) (width 0.25) (layer "F.Cu") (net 9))
 (segment (start 99.527746 71.275819) (end 100.064978 70.738588) (width 0.25) (layer "F.Cu") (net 9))
 (segment (start 100.769464 67.285401) (end 100.769464 63.522336) (width 0.25) (layer "F.Cu") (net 9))
 (segment (start 100.064978 70.738588) (end 100.064978 67.989886) (width 0.25) (layer "F.Cu") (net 9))
 (segment (start 96.995603 74.770999) (end 99.527745 72.238857) (width 0.25) (layer "F.Cu") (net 9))
 (segment (start 100.769464 63.522336) (end 103.5558 60.736) (width 0.25) (layer "F.Cu") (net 9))
 (segment (start 100.319453 63.335937) (end 102.380799 61.274591) (width 0.25) (layer "F.Cu") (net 8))
 (segment (start 96.6216 73.406) (end 99.614967 70.412633) (width 0.25) (layer "F.Cu") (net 8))
 (segment (start 100.319453 67.099001) (end 100.319453 63.335937) (width 0.25) (layer "F.Cu") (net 8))
 (segment (start 102.380799 59.371001) (end 103.5558 58.196) (width 0.25) (layer "F.Cu") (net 8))
 (segment (start 99.614967 70.412633) (end 99.614967 67.803486) (width 0.25) (layer "F.Cu") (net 8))
 (segment (start 102.380799 61.274591) (end 102.380799 59.371001) (width 0.25) (layer "F.Cu") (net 8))
 (segment (start 99.614967 67.803486) (end 100.319453 67.099001) (width 0.25) (layer "F.Cu") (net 8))
 (segment (start 95.256601 72.230999) (end 96.995603 72.230999) (width 0.25) (layer "F.Cu") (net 7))
 (segment (start 99.869442 66.912601) (end 99.869442 63.149537) (width 0.25) (layer "F.Cu") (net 7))
 (segment (start 101.930788 57.281012) (end 103.5558 55.656) (width 0.25) (layer "F.Cu") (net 7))
 (segment (start 96.995603 72.230999) (end 99.164956 70.061646) (width 0.25) (layer "F.Cu") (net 7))
 (segment (start 94.0816 73.406) (end 95.256601 72.230999) (width 0.25) (layer "F.Cu") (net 7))
 (segment (start 99.869442 63.149537) (end 101.930788 61.088191) (width 0.25) (layer "F.Cu") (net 7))
 (segment (start 99.164956 67.617086) (end 99.869442 66.912601) (width 0.25) (layer "F.Cu") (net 7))
 (segment (start 99.164956 70.061646) (end 99.164956 67.617086) (width 0.25) (layer "F.Cu") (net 7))
 (segment (start 101.930788 61.088191) (end 101.930788 57.281012) (width 0.25) (layer "F.Cu") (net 7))
 (segment (start 96.6216 70.866) (end 98.714945 68.772655) (width 0.25) (layer "F.Cu") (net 6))
 (segment (start 101.480777 60.901791) (end 101.480777 55.191023) (width 0.25) (layer "F.Cu") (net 6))
 (segment (start 101.480777 55.191023) (end 102.705801 53.965999) (width 0.25) (layer "F.Cu") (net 6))
 (segment (start 98.714945 67.430686) (end 99.419431 66.726201) (width 0.25) (layer "F.Cu") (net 6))
 (segment (start 98.714945 68.772655) (end 98.714945 67.430686) (width 0.25) (layer "F.Cu") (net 6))
 (segment (start 99.419431 62.963137) (end 101.480777 60.901791) (width 0.25) (layer "F.Cu") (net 6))
 (segment (start 99.419431 66.726201) (end 99.419431 62.963137) (width 0.25) (layer "F.Cu") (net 6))
 (segment (start 102.705801 53.965999) (end 103.5558 53.116) (width 0.25) (layer "F.Cu") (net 6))
 (segment (start 103.5558 50.576) (end 98.96942 55.16238) (width 0.25) (layer "F.Cu") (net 5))
 (segment (start 98.96942 55.16238) (end 98.96942 66.539801) (width 0.25) (layer "F.Cu") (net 5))
 (segment (start 97.141344 69.501001) (end 95.446599 69.501001) (width 0.25) (layer "F.Cu") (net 5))
 (segment (start 95.446599 69.501001) (end 94.0816 70.866) (width 0.25) (layer "F.Cu") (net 5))
 (segment (start 98.264934 68.377412) (end 97.141344 69.501001) (width 0.25) (layer "F.Cu") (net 5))
 (segment (start 98.96942 66.539801) (end 98.264934 67.244286) (width 0.25) (layer "F.Cu") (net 5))
 (segment (start 98.264934 67.244286) (end 98.264934 68.377412) (width 0.25) (layer "F.Cu") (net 5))
 (segment (start 98.519409 66.353401) (end 96.6216 68.25121) (width 0.25) (layer "F.Cu") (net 4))
 (segment (start 98.519409 53.072391) (end 98.519409 66.353401) (width 0.25) (layer "F.Cu") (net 4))
 (segment (start 96.6216 68.25121) (end 96.6216 68.326) (width 0.25) (layer "F.Cu") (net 4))
 (segment (start 103.5558 48.036) (end 98.519409 53.072391) (width 0.25) (layer "F.Cu") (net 4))
 (segment (start 96.247597 66.961001) (end 97.275399 66.961001) (width 0.25) (layer "F.Cu") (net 3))
 (segment (start 95.0976 68.326) (end 95.0976 68.110998) (width 0.25) (layer "F.Cu") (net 3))
 (segment (start 97.275399 66.961001) (end 97.796601 66.439799) (width 0.25) (layer "F.Cu") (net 3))
 (segment (start 95.0976 68.110998) (end 96.247597 66.961001) (width 0.25) (layer "F.Cu") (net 3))
 (segment (start 94.0816 68.326) (end 95.0976 68.326) (width 0.25) (layer "F.Cu") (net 3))
 (segment (start 97.796601 66.439799) (end 97.796601 51.255199) (width 0.25) (layer "F.Cu") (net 3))
 (segment (start 97.796601 51.255199) (end 103.5558 45.496) (width 0.25) (layer "F.Cu") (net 3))
 (segment (start 96.6216 65.786) (end 96.6216 50.691198) (width 0.25) (layer "F.Cu") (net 2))
 (segment (start 103.5558 43.756998) (end 103.5558 42.956) (width 0.25) (layer "F.Cu") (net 2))
 (segment (start 96.6216 50.691198) (end 103.5558 43.756998) (width 0.25) (layer "F.Cu") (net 2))
 (segment (start 94.0816 49.8902) (end 94.0816 65.786) (width 0.25) (layer "F.Cu") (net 1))
 (segment (start 103.5558 40.416) (end 94.0816 49.8902) (width 0.25) (layer "F.Cu") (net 1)))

